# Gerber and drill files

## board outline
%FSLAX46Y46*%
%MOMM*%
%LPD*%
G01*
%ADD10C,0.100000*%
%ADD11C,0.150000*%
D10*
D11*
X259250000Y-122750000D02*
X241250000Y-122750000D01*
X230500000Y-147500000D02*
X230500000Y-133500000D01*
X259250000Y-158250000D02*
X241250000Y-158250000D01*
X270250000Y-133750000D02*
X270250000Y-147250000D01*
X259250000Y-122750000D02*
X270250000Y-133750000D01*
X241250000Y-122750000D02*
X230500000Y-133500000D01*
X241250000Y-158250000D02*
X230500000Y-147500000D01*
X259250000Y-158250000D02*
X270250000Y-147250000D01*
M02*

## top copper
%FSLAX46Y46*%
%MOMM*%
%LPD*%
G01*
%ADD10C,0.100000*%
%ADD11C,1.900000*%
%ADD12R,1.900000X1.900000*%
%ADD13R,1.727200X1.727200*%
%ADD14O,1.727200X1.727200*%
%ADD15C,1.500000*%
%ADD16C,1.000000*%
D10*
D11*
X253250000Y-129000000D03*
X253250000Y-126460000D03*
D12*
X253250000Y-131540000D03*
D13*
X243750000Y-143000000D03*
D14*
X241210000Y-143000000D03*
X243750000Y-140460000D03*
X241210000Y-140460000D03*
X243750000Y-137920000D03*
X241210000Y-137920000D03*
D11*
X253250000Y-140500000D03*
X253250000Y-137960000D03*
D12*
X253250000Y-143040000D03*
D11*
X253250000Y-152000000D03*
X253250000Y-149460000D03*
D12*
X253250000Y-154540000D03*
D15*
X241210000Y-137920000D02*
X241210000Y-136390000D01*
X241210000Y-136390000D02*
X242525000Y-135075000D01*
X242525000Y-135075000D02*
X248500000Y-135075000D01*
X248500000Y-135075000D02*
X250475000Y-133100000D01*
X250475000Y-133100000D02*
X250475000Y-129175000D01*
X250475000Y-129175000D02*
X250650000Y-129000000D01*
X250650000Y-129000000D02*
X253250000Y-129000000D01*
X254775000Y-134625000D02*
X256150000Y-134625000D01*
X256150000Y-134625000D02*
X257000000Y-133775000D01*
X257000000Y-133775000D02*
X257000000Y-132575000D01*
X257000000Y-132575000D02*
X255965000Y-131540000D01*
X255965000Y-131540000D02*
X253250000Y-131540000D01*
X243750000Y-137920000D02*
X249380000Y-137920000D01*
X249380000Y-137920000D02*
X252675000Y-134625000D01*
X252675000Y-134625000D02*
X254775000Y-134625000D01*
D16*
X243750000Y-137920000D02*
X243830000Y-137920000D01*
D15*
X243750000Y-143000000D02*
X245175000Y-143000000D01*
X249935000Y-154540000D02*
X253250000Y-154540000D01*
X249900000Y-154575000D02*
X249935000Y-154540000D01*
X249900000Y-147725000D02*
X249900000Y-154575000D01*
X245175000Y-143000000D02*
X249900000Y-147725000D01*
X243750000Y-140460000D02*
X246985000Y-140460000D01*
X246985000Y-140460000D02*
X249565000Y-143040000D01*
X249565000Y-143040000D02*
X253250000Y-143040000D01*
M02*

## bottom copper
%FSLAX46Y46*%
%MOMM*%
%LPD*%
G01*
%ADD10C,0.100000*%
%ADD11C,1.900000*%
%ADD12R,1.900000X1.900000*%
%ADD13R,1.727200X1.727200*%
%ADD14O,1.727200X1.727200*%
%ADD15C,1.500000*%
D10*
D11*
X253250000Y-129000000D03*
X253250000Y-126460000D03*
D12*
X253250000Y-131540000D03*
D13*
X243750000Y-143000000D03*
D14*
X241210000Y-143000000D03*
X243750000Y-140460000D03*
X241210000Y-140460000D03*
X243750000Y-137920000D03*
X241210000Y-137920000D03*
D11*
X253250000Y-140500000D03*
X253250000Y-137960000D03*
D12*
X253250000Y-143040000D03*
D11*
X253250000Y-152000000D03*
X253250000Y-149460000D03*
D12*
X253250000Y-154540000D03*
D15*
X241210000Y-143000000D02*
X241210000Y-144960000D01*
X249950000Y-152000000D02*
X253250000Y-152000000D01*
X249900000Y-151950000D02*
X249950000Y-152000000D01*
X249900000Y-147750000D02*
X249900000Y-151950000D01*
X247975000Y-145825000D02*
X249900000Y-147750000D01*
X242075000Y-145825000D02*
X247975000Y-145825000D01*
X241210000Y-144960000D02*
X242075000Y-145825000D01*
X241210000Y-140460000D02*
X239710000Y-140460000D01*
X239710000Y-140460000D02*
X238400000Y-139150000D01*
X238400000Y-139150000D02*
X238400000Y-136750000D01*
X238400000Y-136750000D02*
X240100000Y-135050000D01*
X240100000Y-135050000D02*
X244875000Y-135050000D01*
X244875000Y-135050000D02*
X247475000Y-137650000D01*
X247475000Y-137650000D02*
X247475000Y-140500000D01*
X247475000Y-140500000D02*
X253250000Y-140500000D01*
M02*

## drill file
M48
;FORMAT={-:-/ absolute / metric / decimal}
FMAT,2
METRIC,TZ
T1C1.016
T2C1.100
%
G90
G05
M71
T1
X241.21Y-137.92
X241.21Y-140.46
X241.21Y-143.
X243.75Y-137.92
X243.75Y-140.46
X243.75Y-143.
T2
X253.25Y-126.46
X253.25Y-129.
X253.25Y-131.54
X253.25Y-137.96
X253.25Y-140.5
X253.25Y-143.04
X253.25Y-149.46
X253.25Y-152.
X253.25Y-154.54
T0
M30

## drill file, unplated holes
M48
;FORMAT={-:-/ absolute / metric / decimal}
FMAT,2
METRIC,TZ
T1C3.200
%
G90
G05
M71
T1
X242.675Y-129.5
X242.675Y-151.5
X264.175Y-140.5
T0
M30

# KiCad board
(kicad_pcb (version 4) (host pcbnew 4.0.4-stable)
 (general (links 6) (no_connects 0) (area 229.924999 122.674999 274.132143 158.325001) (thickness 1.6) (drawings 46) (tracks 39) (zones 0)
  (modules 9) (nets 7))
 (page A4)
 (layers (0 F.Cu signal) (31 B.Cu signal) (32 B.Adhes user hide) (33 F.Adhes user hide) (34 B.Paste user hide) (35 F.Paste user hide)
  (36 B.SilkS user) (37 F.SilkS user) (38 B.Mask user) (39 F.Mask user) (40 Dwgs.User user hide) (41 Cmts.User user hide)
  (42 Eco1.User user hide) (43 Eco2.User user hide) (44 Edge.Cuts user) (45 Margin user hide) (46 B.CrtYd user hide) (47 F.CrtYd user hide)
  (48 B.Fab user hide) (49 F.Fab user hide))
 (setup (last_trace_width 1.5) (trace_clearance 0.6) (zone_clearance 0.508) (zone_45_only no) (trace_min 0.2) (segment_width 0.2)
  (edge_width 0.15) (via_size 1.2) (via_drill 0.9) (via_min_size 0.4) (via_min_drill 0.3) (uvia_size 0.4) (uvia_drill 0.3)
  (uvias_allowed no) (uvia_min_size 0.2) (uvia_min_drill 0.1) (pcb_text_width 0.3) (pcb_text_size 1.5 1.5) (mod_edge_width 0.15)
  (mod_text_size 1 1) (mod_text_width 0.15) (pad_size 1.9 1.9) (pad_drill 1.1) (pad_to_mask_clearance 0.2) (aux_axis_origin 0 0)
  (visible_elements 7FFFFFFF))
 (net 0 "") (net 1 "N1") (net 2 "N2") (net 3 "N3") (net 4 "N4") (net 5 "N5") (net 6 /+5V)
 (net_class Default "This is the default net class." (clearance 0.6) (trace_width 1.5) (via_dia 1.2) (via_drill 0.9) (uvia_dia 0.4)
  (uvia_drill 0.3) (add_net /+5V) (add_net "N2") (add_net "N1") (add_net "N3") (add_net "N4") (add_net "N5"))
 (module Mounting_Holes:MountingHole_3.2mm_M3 (layer F.Cu) (at 264.175 140.5)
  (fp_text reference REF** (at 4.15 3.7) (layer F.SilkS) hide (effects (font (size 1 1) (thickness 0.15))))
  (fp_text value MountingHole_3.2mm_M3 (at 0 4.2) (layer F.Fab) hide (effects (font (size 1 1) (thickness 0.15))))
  (pad 1 np_thru_hole circle (at 0 0) (size 3.2 3.2) (drill 3.2) (layers *.Cu *.Mask)))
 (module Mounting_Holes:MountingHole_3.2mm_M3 (layer F.Cu) (at 242.675 151.5)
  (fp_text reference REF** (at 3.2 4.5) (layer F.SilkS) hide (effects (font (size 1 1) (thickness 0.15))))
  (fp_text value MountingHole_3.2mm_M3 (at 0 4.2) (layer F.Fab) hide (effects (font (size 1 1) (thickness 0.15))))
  (pad 1 np_thru_hole circle (at 0 0) (size 3.2 3.2) (drill 3.2) (layers *.Cu *.Mask)))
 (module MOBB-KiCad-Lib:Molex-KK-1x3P (layer B.Cu) (at 253.25 129 270)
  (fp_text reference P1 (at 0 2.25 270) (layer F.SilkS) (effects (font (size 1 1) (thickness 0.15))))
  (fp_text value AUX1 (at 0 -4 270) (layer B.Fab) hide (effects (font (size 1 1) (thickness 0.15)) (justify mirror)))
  (pad 2 thru_hole circle (at 0 0 270) (size 1.9 1.9) (drill 1.1) (layers *.Cu *.Mask) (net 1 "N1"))
  (pad 3 thru_hole circle (at -2.54 0 270) (size 1.9 1.9) (drill 1.1) (layers *.Cu *.Mask))
  (pad 1 thru_hole rect (at 2.54 0 270) (size 1.9 1.9) (drill 1.1) (layers *.Cu *.Mask) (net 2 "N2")))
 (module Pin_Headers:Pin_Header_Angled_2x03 (layer F.Cu) (at 243.75 143 180)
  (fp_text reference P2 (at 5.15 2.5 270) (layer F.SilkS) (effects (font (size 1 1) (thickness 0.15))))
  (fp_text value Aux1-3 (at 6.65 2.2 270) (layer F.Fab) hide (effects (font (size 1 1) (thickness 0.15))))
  (pad 1 thru_hole rect (at 0 0 180) (size 1.7272 1.7272) (drill 1.016) (layers *.Cu *.Mask) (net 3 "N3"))
  (pad 2 thru_hole oval (at 2.54 0 180) (size 1.7272 1.7272) (drill 1.016) (layers *.Cu *.Mask) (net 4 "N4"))
  (pad 3 thru_hole oval (at 0 2.54 180) (size 1.7272 1.7272) (drill 1.016) (layers *.Cu *.Mask) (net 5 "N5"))
  (pad 4 thru_hole oval (at 2.54 2.54 180) (size 1.7272 1.7272) (drill 1.016) (layers *.Cu *.Mask) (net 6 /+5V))
  (pad 5 thru_hole oval (at 0 5.08 180) (size 1.7272 1.7272) (drill 1.016) (layers *.Cu *.Mask) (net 2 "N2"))
  (pad 6 thru_hole oval (at 2.54 5.08 180) (size 1.7272 1.7272) (drill 1.016) (layers *.Cu *.Mask) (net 1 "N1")))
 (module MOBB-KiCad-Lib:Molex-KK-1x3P (layer B.Cu) (at 253.25 140.5 270)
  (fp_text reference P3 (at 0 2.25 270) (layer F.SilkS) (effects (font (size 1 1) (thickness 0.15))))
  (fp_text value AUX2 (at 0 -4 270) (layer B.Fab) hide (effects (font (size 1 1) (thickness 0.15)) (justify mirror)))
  (pad 2 thru_hole circle (at 0 0 270) (size 1.9 1.9) (drill 1.1) (layers *.Cu *.Mask) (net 6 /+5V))
  (pad 3 thru_hole circle (at -2.54 0 270) (size 1.9 1.9) (drill 1.1) (layers *.Cu *.Mask))
  (pad 1 thru_hole rect (at 2.54 0 270) (size 1.9 1.9) (drill 1.1) (layers *.Cu *.Mask) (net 5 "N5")))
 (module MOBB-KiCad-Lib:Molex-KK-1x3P (layer B.Cu) (at 253.25 152 270)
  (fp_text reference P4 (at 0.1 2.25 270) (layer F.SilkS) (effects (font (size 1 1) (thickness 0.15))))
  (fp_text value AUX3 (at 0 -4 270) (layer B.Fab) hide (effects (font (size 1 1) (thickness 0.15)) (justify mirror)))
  (pad 2 thru_hole circle (at 0 0 270) (size 1.9 1.9) (drill 1.1) (layers *.Cu *.Mask) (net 4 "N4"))
  (pad 3 thru_hole circle (at -2.54 0 270) (size 1.9 1.9) (drill 1.1) (layers *.Cu *.Mask))
  (pad 1 thru_hole rect (at 2.54 0 270) (size 1.9 1.9) (drill 1.1) (layers *.Cu *.Mask) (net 3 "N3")))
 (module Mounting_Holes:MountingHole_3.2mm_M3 (layer F.Cu) (at 242.675 129.5)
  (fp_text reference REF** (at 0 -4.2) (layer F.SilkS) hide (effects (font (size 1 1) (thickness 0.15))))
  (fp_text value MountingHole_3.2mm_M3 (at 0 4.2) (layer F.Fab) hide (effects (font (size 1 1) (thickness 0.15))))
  (pad 1 np_thru_hole circle (at 0 0) (size 3.2 3.2) (drill 3.2) (layers *.Cu *.Mask)))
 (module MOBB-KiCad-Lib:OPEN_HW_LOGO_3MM (layer F.Cu) (at 237.1 130.5)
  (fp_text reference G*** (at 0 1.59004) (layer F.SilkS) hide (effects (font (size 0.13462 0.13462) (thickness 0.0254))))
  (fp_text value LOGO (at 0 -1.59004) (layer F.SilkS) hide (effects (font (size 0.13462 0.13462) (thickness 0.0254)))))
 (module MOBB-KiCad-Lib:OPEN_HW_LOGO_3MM (layer B.Cu) (at 237.1 130.5 180)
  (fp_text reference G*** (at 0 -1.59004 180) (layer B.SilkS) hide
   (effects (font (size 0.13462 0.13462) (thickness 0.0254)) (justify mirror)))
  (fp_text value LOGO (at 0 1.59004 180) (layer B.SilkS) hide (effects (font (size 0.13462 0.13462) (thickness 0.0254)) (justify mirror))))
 (gr_line (start 259.25 122.75) (end 241.25 122.75) (angle 90) (layer Edge.Cuts) (width 0.15))
 (gr_line (start 230.5 147.5) (end 230.5 133.5) (angle 90) (layer Edge.Cuts) (width 0.15))
 (gr_line (start 259.25 158.25) (end 241.25 158.25) (angle 90) (layer Edge.Cuts) (width 0.15))
 (gr_line (start 270.25 133.75) (end 270.25 147.25) (angle 90) (layer Edge.Cuts) (width 0.15))
 (gr_line (start 259.25 122.75) (end 270.25 133.75) (angle 90) (layer Edge.Cuts) (width 0.15))
 (gr_line (start 241.25 122.75) (end 230.5 133.5) (angle 90) (layer Edge.Cuts) (width 0.15))
 (gr_line (start 241.25 158.25) (end 230.5 147.5) (angle 90) (layer Edge.Cuts) (width 0.15))
 (gr_line (start 259.25 158.25) (end 270.25 147.25) (angle 90) (layer Edge.Cuts) (width 0.15))
 (segment (start 241.21 137.92) (end 241.21 136.39) (width 1.5) (layer F.Cu) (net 1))
 (segment (start 241.21 136.39) (end 242.525 135.075) (width 1.5) (layer F.Cu) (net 1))
 (segment (start 242.525 135.075) (end 248.5 135.075) (width 1.5) (layer F.Cu) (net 1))
 (segment (start 248.5 135.075) (end 250.475 133.1) (width 1.5) (layer F.Cu) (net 1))
 (segment (start 250.475 133.1) (end 250.475 129.175) (width 1.5) (layer F.Cu) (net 1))
 (segment (start 250.475 129.175) (end 250.65 129) (width 1.5) (layer F.Cu) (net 1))
 (segment (start 250.65 129) (end 253.25 129) (width 1.5) (layer F.Cu) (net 1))
 (segment (start 254.775 134.625) (end 256.15 134.625) (width 1.5) (layer F.Cu) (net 2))
 (segment (start 256.15 134.625) (end 257 133.775) (width 1.5) (layer F.Cu) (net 2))
 (segment (start 257 133.775) (end 257 132.575) (width 1.5) (layer F.Cu) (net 2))
 (segment (start 257 132.575) (end 255.965 131.54) (width 1.5) (layer F.Cu) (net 2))
 (segment (start 255.965 131.54) (end 253.25 131.54) (width 1.5) (layer F.Cu) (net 2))
 (segment (start 243.75 137.92) (end 249.38 137.92) (width 1.5) (layer F.Cu) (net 2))
 (segment (start 249.38 137.92) (end 252.675 134.625) (width 1.5) (layer F.Cu) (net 2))
 (segment (start 252.675 134.625) (end 254.775 134.625) (width 1.5) (layer F.Cu) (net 2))
 (segment (start 243.75 137.92) (end 243.83 137.92) (width 1) (layer F.Cu) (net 2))
 (segment (start 243.75 143) (end 245.175 143) (width 1.5) (layer F.Cu) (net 3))
 (segment (start 249.935 154.54) (end 253.25 154.54) (width 1.5) (layer F.Cu) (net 3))
 (segment (start 249.9 154.575) (end 249.935 154.54) (width 1.5) (layer F.Cu) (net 3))
 (segment (start 249.9 147.725) (end 249.9 154.575) (width 1.5) (layer F.Cu) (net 3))
 (segment (start 245.175 143) (end 249.9 147.725) (width 1.5) (layer F.Cu) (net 3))
 (segment (start 241.21 143) (end 241.21 144.96) (width 1.5) (layer B.Cu) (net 4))
 (segment (start 249.95 152) (end 253.25 152) (width 1.5) (layer B.Cu) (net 4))
 (segment (start 249.9 151.95) (end 249.95 152) (width 1.5) (layer B.Cu) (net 4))
 (segment (start 249.9 147.75) (end 249.9 151.95) (width 1.5) (layer B.Cu) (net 4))
 (segment (start 247.975 145.825) (end 249.9 147.75) (width 1.5) (layer B.Cu) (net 4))
 (segment (start 242.075 145.825) (end 247.975 145.825) (width 1.5) (layer B.Cu) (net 4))
 (segment (start 241.21 144.96) (end 242.075 145.825) (width 1.5) (layer B.Cu) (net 4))
 (segment (start 243.75 140.46) (end 246.985 140.46) (width 1.5) (layer F.Cu) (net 5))
 (segment (start 246.985 140.46) (end 249.565 143.04) (width 1.5) (layer F.Cu) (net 5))
 (segment (start 249.565 143.04) (end 253.25 143.04) (width 1.5) (layer F.Cu) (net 5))
 (segment (start 241.21 140.46) (end 239.71 140.46) (width 1.5) (layer B.Cu) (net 6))
 (segment (start 239.71 140.46) (end 238.4 139.15) (width 1.5) (layer B.Cu) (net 6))
 (segment (start 238.4 139.15) (end 238.4 136.75) (width 1.5) (layer B.Cu) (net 6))
 (segment (start 238.4 136.75) (end 240.1 135.05) (width 1.5) (layer B.Cu) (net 6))
 (segment (start 240.1 135.05) (end 244.875 135.05) (width 1.5) (layer B.Cu) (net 6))
 (segment (start 244.875 135.05) (end 247.475 137.65) (width 1.5) (layer B.Cu) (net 6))
 (segment (start 247.475 137.65) (end 247.475 140.5) (width 1.5) (layer B.Cu) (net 6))
 (segment (start 247.475 140.5) (end 253.25 140.5) (width 1.5) (layer B.Cu) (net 6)))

